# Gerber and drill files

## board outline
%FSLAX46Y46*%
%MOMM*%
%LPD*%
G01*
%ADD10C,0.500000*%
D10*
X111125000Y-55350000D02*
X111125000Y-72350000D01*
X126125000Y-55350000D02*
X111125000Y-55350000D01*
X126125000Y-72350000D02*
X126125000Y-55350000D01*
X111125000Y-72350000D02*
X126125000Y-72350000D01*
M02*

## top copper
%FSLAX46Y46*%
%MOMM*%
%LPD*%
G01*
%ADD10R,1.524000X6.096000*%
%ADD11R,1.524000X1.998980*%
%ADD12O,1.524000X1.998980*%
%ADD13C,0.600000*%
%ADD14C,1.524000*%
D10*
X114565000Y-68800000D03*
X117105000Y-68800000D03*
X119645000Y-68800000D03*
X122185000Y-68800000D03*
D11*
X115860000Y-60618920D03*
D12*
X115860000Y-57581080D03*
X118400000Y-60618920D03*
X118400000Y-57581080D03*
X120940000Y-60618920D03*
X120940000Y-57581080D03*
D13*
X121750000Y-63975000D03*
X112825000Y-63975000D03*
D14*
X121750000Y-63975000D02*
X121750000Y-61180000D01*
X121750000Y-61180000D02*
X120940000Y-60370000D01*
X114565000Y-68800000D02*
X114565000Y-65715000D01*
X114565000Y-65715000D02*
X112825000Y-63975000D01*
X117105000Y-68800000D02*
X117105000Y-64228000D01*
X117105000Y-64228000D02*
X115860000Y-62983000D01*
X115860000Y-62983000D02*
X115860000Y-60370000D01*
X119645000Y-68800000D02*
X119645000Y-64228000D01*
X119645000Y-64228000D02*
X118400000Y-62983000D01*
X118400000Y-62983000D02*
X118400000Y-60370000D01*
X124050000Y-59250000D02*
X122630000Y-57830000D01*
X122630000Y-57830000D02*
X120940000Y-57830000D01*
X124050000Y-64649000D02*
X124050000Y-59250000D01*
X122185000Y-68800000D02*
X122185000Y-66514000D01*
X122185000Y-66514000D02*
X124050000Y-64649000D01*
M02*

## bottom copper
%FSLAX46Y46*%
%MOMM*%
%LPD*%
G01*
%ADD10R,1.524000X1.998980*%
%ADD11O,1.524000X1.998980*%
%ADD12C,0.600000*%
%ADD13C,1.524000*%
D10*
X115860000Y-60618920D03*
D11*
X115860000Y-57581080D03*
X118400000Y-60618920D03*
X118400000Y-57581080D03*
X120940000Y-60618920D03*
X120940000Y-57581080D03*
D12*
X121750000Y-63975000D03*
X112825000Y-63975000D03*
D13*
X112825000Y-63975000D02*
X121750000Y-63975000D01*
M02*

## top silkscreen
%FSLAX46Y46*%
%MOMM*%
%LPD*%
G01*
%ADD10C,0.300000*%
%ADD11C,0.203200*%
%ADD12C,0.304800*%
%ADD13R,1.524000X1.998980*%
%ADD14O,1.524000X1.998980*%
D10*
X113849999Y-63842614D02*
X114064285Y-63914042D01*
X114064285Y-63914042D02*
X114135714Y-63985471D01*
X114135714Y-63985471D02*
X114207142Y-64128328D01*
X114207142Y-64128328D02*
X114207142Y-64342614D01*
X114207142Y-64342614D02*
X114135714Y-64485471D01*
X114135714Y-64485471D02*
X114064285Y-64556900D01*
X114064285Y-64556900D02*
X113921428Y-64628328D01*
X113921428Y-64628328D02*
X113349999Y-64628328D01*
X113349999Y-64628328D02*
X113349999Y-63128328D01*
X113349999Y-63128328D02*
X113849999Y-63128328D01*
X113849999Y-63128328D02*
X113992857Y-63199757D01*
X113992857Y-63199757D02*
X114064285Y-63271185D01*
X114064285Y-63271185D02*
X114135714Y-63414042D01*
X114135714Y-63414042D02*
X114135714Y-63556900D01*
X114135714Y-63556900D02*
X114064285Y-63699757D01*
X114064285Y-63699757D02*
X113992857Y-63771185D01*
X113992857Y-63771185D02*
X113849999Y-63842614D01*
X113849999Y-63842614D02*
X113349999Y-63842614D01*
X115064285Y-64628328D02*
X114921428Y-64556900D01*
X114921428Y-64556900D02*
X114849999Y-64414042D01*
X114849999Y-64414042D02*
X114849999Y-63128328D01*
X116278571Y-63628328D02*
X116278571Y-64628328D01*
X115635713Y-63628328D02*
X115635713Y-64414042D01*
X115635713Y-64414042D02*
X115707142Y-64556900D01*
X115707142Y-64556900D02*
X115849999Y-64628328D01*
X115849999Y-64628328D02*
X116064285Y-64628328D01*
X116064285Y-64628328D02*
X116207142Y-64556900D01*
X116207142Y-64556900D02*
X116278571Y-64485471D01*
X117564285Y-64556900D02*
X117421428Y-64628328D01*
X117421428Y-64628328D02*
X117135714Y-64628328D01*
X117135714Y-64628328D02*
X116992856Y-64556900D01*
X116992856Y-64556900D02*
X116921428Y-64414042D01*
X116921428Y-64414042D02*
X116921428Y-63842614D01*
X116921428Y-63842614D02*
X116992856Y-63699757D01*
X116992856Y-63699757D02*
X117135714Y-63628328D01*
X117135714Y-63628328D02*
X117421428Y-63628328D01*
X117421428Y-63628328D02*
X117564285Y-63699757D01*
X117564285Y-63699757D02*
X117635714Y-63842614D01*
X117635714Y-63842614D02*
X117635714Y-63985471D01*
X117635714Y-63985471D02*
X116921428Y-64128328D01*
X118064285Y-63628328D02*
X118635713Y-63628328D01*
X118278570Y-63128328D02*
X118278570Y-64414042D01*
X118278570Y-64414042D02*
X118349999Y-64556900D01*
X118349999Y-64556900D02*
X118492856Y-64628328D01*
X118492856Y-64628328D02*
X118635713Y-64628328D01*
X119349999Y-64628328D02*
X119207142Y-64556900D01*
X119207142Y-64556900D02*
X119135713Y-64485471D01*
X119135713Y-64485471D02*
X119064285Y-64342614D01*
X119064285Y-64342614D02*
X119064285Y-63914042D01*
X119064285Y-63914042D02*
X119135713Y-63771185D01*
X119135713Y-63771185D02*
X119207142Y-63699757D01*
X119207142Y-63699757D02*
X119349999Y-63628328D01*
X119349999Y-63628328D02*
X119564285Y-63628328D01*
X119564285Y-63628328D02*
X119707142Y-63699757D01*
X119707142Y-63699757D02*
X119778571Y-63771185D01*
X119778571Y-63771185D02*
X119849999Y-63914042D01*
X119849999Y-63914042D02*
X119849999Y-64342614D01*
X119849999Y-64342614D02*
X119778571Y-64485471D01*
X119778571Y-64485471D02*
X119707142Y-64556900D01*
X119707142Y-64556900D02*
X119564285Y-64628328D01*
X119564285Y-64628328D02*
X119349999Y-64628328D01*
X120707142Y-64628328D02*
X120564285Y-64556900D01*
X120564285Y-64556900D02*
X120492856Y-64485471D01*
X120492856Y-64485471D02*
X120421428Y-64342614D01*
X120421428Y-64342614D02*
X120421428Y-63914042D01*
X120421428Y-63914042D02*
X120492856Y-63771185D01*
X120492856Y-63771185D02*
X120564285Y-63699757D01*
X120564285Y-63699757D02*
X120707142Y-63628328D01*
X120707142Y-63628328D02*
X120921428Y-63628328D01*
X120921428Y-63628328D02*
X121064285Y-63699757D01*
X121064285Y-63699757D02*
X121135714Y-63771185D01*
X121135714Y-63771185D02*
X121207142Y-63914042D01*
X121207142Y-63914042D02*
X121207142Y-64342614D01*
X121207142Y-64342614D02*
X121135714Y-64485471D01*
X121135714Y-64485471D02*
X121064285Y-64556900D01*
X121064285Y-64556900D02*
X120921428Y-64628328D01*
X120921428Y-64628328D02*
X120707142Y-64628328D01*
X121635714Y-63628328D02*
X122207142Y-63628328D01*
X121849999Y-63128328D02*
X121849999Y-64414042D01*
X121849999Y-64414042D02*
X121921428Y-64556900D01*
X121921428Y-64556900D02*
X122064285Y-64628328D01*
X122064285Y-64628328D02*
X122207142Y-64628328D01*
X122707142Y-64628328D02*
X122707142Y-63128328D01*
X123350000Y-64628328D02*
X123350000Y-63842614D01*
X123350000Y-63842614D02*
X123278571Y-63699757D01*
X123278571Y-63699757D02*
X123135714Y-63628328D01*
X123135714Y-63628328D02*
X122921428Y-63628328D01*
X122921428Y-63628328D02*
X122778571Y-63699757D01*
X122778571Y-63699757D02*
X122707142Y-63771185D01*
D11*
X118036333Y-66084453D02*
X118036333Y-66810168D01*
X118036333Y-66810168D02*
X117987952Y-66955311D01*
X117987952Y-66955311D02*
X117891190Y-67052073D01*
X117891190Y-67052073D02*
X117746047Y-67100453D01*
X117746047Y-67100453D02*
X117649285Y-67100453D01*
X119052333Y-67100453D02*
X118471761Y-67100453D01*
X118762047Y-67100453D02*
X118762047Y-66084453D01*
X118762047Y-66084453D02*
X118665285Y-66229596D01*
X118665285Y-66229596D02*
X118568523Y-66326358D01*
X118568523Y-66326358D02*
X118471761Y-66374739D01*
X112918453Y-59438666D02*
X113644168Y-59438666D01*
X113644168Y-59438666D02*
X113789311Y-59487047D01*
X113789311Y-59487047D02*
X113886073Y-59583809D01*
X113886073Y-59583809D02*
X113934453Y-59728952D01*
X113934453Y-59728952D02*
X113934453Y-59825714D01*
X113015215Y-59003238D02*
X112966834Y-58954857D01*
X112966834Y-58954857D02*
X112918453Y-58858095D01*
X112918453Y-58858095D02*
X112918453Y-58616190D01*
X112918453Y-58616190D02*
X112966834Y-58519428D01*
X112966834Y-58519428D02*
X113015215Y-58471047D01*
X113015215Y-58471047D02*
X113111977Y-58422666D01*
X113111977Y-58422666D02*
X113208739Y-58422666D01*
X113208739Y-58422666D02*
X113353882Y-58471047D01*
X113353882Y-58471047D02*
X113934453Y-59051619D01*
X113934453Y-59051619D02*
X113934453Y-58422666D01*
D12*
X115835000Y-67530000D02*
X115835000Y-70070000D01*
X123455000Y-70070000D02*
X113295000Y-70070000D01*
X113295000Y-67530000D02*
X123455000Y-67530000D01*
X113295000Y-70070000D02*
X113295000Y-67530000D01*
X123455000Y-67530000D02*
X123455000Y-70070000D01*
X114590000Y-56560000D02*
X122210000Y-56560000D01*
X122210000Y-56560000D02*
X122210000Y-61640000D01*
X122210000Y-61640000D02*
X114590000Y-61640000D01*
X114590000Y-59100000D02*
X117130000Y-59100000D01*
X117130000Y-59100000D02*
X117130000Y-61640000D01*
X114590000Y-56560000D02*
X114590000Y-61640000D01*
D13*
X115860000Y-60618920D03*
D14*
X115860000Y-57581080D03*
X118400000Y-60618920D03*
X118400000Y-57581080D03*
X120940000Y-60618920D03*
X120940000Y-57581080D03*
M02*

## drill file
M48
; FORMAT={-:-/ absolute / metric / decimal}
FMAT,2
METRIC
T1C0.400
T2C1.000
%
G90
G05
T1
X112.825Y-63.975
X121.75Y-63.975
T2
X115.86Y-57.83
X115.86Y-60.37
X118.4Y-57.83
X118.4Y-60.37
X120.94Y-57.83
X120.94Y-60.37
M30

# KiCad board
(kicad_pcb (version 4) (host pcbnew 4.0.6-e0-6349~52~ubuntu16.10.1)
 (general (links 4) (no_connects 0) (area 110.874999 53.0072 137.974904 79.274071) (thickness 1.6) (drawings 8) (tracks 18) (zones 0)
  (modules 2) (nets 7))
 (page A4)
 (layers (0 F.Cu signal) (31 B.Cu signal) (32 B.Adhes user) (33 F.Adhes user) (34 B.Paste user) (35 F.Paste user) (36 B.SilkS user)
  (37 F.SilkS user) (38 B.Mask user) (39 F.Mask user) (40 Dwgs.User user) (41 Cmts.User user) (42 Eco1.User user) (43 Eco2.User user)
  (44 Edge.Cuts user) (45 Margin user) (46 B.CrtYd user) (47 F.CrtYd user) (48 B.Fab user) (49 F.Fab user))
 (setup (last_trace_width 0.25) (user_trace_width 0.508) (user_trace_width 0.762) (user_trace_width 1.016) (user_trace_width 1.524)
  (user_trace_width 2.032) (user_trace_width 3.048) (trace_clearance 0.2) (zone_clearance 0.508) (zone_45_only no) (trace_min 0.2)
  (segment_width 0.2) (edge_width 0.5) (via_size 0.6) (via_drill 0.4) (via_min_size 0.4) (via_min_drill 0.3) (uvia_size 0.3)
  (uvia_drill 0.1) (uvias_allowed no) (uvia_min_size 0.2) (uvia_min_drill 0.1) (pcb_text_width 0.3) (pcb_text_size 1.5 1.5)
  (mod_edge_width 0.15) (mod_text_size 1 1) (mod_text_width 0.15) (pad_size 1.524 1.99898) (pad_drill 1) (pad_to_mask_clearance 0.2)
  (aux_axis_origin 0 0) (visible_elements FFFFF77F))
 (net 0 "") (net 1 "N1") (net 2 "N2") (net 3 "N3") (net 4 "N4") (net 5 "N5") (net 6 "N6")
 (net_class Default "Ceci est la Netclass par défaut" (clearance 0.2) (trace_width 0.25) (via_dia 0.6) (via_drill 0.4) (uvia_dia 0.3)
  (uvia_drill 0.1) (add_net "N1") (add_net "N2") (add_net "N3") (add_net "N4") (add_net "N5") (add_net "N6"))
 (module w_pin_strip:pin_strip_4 (layer F.Cu) (at 118.375 68.8)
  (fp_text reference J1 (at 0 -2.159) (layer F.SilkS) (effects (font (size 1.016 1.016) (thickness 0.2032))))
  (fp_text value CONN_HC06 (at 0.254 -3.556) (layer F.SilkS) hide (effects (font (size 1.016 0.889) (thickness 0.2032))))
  (fp_line (start -2.54 -1.27) (end -2.54 1.27) (layer F.SilkS) (width 0.3048))
  (fp_line (start 5.08 1.27) (end -5.08 1.27) (layer F.SilkS) (width 0.3048))
  (fp_line (start -5.08 -1.27) (end 5.08 -1.27) (layer F.SilkS) (width 0.3048))
  (fp_line (start -5.08 1.27) (end -5.08 -1.27) (layer F.SilkS) (width 0.3048))
  (fp_line (start 5.08 -1.27) (end 5.08 1.27) (layer F.SilkS) (width 0.3048))
  (pad 1 smd rect (at -3.81 0) (size 1.524 6.096) (layers F.Cu F.Paste F.Mask) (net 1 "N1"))
  (pad 2 smd rect (at -1.27 0) (size 1.524 6.096) (layers F.Cu F.Paste F.Mask) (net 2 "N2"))
  (pad 3 smd rect (at 1.27 0) (size 1.524 6.096) (layers F.Cu F.Paste F.Mask) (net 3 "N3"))
  (pad 4 smd rect (at 3.81 0) (size 1.524 6.096) (layers F.Cu F.Paste F.Mask) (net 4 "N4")))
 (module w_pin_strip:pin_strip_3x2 (layer F.Cu) (at 118.4 59.1)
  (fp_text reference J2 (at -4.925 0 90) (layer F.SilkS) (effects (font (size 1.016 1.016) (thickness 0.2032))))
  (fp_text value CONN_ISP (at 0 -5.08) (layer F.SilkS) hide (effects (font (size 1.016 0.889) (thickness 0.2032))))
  (fp_line (start -3.81 -2.54) (end 3.81 -2.54) (layer F.SilkS) (width 0.3048))
  (fp_line (start 3.81 -2.54) (end 3.81 2.54) (layer F.SilkS) (width 0.3048))
  (fp_line (start 3.81 2.54) (end -3.81 2.54) (layer F.SilkS) (width 0.3048))
  (fp_line (start -3.81 0) (end -1.27 0) (layer F.SilkS) (width 0.3048))
  (fp_line (start -1.27 0) (end -1.27 2.54) (layer F.SilkS) (width 0.3048))
  (fp_line (start -3.81 -2.54) (end -3.81 2.54) (layer F.SilkS) (width 0.3048))
  (pad 1 thru_hole rect (at -2.54 1.27) (size 1.524 1.99898) (drill 1 (offset 0 0.24892)) (layers *.Cu *.Mask F.SilkS) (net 2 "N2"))
  (pad 2 thru_hole oval (at -2.54 -1.27) (size 1.524 1.99898) (drill 1 (offset 0 -0.24892)) (layers *.Cu *.Mask F.SilkS) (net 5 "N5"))
  (pad 3 thru_hole oval (at 0 1.27) (size 1.524 1.99898) (drill 1 (offset 0 0.24892)) (layers *.Cu *.Mask F.SilkS) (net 3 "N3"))
  (pad 4 thru_hole oval (at 0 -1.27) (size 1.524 1.99898) (drill 1 (offset 0 -0.24892)) (layers *.Cu *.Mask F.SilkS) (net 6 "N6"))
  (pad 5 thru_hole oval (at 2.54 1.27) (size 1.524 1.99898) (drill 1 (offset 0 0.24892)) (layers *.Cu *.Mask F.SilkS) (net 1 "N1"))
  (pad 6 thru_hole oval (at 2.54 -1.27) (size 1.524 1.99898) (drill 1 (offset 0 -0.24892)) (layers *.Cu *.Mask F.SilkS) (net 4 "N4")))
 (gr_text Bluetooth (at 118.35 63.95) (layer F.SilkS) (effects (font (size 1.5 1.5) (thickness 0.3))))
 (gr_line (start 111.125 55.35) (end 111.125 72.35) (layer Edge.Cuts) (width 0.5))
 (gr_line (start 126.125 55.35) (end 111.125 55.35) (layer Edge.Cuts) (width 0.5))
 (gr_line (start 126.125 72.35) (end 126.125 55.35) (layer Edge.Cuts) (width 0.5))
 (gr_line (start 111.125 72.35) (end 126.125 72.35) (layer Edge.Cuts) (width 0.5))
 (segment (start 121.75 63.975) (end 121.75 61.18) (width 1.524) (layer F.Cu) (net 1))
 (segment (start 121.75 61.18) (end 120.94 60.37) (width 1.524) (layer F.Cu) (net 1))
 (segment (start 112.825 63.975) (end 121.75 63.975) (width 1.524) (layer B.Cu) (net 1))
 (via (at 121.75 63.975) (size 0.6) (drill 0.4) (layers F.Cu B.Cu) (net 1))
 (segment (start 114.565 68.8) (end 114.565 65.715) (width 1.524) (layer F.Cu) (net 1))
 (segment (start 114.565 65.715) (end 112.825 63.975) (width 1.524) (layer F.Cu) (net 1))
 (via (at 112.825 63.975) (size 0.6) (drill 0.4) (layers F.Cu B.Cu) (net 1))
 (segment (start 117.105 68.8) (end 117.105 64.228) (width 1.524) (layer F.Cu) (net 2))
 (segment (start 117.105 64.228) (end 115.86 62.983) (width 1.524) (layer F.Cu) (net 2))
 (segment (start 115.86 62.983) (end 115.86 60.37) (width 1.524) (layer F.Cu) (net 2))
 (segment (start 119.645 68.8) (end 119.645 64.228) (width 1.524) (layer F.Cu) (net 3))
 (segment (start 119.645 64.228) (end 118.4 62.983) (width 1.524) (layer F.Cu) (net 3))
 (segment (start 118.4 62.983) (end 118.4 60.37) (width 1.524) (layer F.Cu) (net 3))
 (segment (start 124.05 59.25) (end 122.63 57.83) (width 1.524) (layer F.Cu) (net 4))
 (segment (start 122.63 57.83) (end 120.94 57.83) (width 1.524) (layer F.Cu) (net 4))
 (segment (start 124.05 64.649) (end 124.05 59.25) (width 1.524) (layer F.Cu) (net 4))
 (segment (start 122.185 68.8) (end 122.185 66.514) (width 1.524) (layer F.Cu) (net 4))
 (segment (start 122.185 66.514) (end 124.05 64.649) (width 1.524) (layer F.Cu) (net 4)))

